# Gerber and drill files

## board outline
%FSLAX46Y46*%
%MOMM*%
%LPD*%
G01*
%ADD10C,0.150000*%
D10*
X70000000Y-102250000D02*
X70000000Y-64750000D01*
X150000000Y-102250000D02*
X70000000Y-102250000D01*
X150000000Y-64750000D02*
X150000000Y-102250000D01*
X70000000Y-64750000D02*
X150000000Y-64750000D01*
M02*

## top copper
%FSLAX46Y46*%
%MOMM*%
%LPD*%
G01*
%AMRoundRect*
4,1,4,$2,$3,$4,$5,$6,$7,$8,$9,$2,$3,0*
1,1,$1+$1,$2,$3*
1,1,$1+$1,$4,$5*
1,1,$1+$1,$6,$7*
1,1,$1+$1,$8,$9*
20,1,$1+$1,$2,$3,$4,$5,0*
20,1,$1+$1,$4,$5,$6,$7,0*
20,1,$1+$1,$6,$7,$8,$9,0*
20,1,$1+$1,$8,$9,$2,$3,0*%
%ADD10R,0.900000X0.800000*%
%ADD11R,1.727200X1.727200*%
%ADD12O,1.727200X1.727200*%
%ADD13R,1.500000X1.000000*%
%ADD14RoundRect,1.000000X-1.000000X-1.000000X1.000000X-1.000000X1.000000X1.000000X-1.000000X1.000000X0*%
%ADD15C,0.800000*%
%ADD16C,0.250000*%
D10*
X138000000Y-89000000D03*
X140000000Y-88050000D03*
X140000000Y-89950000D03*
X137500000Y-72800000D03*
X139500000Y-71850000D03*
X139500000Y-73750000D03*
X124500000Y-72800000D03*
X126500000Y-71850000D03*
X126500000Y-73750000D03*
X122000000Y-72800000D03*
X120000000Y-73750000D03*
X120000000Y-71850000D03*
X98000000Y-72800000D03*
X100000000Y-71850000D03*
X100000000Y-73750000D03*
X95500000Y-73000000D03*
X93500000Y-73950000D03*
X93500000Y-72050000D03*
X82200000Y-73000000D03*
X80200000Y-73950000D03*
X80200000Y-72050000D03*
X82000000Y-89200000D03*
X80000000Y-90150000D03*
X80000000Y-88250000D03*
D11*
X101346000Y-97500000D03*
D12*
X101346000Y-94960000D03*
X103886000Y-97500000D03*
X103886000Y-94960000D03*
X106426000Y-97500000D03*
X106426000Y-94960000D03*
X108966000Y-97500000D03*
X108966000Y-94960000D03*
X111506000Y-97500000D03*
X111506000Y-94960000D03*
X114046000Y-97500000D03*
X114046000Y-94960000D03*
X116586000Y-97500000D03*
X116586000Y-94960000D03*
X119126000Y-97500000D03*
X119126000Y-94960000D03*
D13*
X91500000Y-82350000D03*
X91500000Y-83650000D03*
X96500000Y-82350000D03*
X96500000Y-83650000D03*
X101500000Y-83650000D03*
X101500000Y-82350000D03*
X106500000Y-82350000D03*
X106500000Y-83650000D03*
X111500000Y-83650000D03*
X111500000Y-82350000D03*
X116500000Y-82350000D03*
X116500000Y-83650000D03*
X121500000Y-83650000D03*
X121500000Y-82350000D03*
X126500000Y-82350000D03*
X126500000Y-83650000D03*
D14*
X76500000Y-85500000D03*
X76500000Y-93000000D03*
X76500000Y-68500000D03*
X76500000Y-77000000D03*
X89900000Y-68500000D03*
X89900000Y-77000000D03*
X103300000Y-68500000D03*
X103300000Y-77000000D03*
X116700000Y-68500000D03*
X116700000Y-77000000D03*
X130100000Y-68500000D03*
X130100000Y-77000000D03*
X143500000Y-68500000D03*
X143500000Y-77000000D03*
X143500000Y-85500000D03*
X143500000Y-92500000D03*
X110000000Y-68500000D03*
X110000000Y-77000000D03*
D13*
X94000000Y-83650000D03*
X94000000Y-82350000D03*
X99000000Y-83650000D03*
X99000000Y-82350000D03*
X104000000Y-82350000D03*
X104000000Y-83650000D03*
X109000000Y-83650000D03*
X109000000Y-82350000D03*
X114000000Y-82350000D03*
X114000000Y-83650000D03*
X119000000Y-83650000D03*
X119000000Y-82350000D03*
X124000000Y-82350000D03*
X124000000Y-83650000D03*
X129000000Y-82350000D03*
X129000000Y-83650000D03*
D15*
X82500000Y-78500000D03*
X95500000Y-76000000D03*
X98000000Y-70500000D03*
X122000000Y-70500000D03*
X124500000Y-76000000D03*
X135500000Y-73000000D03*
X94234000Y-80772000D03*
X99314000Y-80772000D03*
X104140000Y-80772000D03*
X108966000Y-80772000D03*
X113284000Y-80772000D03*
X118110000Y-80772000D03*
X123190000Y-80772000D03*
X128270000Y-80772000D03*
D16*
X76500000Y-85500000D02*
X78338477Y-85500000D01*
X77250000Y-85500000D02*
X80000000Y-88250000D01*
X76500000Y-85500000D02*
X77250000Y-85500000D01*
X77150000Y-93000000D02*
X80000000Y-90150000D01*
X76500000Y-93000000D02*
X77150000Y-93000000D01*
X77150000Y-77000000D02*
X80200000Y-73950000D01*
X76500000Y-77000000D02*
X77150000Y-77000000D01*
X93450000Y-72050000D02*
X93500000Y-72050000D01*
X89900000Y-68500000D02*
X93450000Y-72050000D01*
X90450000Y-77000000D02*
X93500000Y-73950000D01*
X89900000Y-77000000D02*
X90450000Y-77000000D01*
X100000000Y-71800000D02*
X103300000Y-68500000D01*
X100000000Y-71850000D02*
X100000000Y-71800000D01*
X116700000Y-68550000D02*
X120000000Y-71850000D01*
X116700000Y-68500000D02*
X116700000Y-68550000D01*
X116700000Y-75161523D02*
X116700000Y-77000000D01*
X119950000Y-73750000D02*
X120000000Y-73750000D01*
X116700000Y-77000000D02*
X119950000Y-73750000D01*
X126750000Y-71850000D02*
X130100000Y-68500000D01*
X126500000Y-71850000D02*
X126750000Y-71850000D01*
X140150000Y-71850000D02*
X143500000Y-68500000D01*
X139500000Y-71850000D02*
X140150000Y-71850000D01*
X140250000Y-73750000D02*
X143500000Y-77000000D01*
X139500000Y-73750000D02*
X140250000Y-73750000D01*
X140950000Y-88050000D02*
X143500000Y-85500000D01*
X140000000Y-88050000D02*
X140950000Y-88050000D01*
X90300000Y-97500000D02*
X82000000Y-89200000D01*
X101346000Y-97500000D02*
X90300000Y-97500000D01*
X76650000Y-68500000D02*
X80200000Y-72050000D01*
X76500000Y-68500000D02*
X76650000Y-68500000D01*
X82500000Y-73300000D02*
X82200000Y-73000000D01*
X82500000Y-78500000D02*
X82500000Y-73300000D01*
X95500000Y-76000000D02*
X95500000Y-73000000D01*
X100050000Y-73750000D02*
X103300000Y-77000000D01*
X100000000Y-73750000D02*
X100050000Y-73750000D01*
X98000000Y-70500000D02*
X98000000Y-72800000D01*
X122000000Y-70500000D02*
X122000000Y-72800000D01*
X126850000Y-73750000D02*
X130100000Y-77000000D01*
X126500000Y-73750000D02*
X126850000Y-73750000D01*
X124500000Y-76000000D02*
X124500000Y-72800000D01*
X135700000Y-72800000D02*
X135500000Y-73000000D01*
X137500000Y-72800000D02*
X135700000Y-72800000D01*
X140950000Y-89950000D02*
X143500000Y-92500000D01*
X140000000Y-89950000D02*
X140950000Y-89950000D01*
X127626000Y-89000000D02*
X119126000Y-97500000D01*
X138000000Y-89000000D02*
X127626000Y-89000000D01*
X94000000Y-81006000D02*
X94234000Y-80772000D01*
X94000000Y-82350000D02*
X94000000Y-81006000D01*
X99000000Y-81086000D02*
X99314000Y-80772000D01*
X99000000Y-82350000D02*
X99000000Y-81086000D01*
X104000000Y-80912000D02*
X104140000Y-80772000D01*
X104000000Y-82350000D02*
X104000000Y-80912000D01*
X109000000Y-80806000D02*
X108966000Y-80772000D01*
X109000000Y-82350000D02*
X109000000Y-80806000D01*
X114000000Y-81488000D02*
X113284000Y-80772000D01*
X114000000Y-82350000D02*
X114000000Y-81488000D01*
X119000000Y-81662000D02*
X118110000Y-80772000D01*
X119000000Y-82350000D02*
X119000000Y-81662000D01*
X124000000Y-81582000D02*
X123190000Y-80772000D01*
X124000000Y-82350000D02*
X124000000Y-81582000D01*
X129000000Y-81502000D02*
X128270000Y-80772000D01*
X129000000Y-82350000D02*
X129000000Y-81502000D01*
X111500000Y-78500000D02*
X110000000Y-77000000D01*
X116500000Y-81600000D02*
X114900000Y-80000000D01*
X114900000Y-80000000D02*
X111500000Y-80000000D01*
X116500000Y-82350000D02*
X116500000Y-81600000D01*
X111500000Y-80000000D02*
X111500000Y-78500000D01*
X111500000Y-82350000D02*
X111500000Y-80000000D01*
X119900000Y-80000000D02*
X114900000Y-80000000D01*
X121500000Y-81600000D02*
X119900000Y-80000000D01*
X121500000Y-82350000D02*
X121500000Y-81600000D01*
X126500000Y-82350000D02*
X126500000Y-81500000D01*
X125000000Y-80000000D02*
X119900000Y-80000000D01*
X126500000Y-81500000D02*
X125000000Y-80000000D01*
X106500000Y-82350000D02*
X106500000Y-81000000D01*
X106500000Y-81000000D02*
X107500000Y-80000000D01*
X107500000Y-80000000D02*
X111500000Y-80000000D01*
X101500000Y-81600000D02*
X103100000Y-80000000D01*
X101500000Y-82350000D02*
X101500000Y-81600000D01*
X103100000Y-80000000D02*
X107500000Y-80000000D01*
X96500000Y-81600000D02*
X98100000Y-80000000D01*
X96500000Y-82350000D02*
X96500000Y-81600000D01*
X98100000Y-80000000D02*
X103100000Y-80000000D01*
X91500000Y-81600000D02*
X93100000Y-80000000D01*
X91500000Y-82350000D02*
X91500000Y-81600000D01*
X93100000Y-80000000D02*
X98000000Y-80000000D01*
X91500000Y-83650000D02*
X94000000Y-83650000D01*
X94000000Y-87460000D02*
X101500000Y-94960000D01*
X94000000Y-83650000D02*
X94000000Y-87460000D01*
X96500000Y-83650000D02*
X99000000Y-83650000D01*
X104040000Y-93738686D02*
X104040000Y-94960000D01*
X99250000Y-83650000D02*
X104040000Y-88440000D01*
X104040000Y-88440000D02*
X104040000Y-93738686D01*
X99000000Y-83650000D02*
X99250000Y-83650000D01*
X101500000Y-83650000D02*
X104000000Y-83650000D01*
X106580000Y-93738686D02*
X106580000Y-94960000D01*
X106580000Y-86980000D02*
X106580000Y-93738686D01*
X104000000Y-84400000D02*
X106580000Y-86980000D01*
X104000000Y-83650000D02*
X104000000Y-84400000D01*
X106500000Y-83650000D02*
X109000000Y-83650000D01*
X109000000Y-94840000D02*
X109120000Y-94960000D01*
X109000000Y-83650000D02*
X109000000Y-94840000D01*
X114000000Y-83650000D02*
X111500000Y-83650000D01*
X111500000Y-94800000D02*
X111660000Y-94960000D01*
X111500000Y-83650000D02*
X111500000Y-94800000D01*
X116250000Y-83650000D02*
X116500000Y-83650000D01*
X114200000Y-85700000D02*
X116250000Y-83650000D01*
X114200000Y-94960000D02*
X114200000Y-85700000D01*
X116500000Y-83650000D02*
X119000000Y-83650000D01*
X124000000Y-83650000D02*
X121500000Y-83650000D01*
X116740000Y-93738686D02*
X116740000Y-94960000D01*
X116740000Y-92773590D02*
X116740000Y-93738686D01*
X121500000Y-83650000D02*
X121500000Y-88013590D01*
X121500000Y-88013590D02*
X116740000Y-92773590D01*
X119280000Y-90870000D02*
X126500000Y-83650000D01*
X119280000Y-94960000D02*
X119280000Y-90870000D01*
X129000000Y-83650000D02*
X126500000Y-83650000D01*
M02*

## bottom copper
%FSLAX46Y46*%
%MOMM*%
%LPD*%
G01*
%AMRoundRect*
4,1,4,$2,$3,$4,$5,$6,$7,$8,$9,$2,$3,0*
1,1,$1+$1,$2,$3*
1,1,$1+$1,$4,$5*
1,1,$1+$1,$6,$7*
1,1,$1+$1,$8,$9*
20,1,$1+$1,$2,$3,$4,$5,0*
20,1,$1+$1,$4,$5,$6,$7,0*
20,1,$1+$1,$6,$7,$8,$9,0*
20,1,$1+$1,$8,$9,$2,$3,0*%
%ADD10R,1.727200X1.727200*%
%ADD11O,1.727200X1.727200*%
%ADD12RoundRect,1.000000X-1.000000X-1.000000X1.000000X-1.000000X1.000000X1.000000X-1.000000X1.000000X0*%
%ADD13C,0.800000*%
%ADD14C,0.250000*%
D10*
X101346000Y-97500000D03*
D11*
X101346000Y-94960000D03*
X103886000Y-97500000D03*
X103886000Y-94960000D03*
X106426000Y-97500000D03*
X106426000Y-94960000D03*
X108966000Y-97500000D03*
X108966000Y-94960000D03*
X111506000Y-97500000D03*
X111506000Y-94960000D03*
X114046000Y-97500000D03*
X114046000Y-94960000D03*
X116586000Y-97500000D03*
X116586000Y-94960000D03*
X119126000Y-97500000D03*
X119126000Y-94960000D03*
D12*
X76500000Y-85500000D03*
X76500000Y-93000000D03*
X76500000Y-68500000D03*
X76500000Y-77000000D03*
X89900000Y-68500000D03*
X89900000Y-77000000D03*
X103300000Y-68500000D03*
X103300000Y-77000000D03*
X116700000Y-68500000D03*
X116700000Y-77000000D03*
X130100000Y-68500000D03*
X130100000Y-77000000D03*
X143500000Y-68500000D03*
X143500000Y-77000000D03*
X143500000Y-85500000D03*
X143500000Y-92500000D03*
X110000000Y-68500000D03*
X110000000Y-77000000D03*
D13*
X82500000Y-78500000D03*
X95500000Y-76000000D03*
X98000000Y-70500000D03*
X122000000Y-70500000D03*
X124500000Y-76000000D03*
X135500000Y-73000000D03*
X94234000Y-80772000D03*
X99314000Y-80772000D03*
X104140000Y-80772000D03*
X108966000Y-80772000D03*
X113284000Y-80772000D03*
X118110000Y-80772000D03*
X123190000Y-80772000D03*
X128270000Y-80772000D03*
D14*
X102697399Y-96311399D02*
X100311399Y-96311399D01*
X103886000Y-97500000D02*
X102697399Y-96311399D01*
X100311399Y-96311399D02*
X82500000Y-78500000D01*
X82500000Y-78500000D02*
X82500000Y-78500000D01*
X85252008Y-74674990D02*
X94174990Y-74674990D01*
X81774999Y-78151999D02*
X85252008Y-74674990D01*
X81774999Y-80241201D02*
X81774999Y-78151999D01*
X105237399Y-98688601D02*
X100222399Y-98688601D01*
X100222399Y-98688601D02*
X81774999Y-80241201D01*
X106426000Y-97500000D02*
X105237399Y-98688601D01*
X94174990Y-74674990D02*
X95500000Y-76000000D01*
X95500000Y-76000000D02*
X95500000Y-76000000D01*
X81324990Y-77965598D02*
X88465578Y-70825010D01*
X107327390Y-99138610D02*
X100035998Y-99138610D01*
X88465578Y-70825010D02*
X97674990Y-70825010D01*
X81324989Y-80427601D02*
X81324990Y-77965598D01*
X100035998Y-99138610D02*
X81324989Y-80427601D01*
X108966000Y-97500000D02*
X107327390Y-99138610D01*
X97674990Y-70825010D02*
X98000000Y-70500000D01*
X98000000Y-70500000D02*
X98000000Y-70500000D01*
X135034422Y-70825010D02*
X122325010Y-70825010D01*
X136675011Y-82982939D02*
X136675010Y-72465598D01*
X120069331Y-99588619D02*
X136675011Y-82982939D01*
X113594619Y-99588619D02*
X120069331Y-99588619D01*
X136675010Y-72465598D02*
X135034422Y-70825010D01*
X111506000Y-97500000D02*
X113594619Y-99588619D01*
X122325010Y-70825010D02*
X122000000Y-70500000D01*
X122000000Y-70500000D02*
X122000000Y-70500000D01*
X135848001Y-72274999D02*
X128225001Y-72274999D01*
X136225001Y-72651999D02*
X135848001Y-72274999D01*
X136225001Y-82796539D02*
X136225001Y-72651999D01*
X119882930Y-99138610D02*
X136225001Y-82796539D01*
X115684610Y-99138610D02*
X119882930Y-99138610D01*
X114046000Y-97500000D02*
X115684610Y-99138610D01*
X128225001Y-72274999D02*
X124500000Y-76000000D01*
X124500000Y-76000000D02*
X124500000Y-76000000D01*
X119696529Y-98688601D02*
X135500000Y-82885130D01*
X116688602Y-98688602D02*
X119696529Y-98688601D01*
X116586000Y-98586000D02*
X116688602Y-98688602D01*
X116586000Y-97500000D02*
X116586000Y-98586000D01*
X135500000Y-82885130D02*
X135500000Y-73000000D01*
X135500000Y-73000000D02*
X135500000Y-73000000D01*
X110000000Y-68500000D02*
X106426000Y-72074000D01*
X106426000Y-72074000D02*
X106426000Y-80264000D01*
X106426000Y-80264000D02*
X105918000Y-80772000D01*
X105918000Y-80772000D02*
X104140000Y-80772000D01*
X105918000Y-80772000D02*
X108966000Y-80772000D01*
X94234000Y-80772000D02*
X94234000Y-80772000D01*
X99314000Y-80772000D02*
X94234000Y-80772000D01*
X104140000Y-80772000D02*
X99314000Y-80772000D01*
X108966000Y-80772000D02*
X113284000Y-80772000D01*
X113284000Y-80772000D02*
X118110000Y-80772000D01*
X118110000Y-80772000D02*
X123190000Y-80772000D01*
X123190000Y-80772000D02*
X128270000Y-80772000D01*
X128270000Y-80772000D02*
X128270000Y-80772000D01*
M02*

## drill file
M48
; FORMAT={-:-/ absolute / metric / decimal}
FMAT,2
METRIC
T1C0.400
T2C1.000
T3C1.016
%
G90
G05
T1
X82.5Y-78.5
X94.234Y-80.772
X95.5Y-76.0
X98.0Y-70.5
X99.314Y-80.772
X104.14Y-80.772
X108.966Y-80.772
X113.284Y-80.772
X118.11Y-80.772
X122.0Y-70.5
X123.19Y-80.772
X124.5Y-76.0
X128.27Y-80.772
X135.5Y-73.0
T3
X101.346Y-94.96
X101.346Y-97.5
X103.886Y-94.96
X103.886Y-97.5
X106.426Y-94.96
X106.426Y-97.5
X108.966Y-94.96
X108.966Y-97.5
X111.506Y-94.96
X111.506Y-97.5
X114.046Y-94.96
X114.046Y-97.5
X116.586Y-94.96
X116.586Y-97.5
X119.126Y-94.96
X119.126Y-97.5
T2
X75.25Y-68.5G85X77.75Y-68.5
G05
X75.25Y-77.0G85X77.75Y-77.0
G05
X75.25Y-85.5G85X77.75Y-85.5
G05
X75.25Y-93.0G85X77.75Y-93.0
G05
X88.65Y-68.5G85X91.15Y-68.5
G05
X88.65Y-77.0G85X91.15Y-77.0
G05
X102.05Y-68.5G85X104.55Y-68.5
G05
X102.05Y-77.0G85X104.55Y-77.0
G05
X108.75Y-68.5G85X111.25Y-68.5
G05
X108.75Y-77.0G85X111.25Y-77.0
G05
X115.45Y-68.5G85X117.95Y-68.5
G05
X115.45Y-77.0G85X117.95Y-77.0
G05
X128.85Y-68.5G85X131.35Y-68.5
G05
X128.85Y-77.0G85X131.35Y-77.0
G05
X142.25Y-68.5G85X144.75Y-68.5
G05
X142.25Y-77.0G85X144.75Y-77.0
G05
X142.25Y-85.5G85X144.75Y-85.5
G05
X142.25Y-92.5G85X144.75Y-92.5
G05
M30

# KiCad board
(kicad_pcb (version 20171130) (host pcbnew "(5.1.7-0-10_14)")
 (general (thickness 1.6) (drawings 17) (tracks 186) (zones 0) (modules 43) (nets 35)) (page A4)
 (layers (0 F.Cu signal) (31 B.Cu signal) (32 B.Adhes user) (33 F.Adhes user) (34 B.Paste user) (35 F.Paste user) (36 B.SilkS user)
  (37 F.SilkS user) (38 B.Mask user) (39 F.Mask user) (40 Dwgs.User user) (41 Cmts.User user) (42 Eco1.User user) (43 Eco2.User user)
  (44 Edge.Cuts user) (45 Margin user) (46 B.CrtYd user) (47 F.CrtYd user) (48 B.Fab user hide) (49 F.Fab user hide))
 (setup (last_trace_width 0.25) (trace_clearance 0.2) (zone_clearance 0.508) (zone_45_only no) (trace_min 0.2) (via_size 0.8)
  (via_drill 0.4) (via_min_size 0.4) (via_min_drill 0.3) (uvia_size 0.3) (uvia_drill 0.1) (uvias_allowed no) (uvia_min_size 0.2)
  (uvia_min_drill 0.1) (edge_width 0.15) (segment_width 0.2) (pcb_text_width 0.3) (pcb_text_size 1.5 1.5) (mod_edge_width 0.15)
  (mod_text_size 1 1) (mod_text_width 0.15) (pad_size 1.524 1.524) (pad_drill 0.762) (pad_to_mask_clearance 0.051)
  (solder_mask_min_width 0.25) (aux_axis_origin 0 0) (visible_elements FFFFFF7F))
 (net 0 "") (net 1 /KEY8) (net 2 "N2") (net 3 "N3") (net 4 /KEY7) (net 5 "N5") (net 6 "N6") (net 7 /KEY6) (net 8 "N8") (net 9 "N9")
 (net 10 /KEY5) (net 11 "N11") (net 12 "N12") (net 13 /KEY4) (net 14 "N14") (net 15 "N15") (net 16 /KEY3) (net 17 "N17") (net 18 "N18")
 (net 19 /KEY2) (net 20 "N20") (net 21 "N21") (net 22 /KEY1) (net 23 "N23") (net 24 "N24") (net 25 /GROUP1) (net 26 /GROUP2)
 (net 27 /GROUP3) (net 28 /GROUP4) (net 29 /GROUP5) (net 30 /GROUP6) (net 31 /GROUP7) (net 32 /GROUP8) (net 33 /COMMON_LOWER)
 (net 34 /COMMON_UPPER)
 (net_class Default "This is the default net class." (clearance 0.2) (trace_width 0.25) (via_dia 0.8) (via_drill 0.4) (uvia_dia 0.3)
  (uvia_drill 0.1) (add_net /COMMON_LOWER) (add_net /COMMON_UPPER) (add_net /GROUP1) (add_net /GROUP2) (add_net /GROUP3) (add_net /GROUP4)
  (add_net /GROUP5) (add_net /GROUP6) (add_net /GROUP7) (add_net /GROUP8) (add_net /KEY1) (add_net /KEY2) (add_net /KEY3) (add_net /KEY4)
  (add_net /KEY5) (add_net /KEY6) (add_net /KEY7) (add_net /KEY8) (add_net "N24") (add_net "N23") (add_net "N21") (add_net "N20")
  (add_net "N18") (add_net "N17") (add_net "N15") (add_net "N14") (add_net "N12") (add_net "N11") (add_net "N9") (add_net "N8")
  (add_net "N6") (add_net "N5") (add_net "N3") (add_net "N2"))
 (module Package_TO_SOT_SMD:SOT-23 (layer F.Cu) (at 139 89 180)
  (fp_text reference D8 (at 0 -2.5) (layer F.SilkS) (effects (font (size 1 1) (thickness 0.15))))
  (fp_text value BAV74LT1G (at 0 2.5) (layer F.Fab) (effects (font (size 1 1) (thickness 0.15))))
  (pad 3 smd rect (at 1 0 180) (size 0.9 0.8) (layers F.Cu F.Paste F.Mask) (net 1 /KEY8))
  (pad 2 smd rect (at -1 0.95 180) (size 0.9 0.8) (layers F.Cu F.Paste F.Mask) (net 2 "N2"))
  (pad 1 smd rect (at -1 -0.95 180) (size 0.9 0.8) (layers F.Cu F.Paste F.Mask) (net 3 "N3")))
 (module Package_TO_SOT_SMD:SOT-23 (layer F.Cu) (at 138.5 72.8 180)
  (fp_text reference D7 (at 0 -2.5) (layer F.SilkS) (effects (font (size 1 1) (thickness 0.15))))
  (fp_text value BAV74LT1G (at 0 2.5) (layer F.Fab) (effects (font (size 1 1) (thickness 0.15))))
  (pad 3 smd rect (at 1 0 180) (size 0.9 0.8) (layers F.Cu F.Paste F.Mask) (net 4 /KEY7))
  (pad 2 smd rect (at -1 0.95 180) (size 0.9 0.8) (layers F.Cu F.Paste F.Mask) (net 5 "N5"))
  (pad 1 smd rect (at -1 -0.95 180) (size 0.9 0.8) (layers F.Cu F.Paste F.Mask) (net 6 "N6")))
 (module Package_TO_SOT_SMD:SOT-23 (layer F.Cu) (at 125.5 72.8 180)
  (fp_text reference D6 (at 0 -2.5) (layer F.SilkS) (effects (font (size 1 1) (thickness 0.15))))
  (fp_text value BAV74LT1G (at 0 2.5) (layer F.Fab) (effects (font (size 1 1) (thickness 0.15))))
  (pad 3 smd rect (at 1 0 180) (size 0.9 0.8) (layers F.Cu F.Paste F.Mask) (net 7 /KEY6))
  (pad 2 smd rect (at -1 0.95 180) (size 0.9 0.8) (layers F.Cu F.Paste F.Mask) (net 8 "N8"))
  (pad 1 smd rect (at -1 -0.95 180) (size 0.9 0.8) (layers F.Cu F.Paste F.Mask) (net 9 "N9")))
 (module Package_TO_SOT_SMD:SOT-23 (layer F.Cu) (at 121 72.8)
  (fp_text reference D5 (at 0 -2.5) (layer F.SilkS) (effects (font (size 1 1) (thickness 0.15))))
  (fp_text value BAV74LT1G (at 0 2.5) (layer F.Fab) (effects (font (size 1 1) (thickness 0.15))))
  (pad 3 smd rect (at 1 0) (size 0.9 0.8) (layers F.Cu F.Paste F.Mask) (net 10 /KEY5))
  (pad 2 smd rect (at -1 0.95) (size 0.9 0.8) (layers F.Cu F.Paste F.Mask) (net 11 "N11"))
  (pad 1 smd rect (at -1 -0.95) (size 0.9 0.8) (layers F.Cu F.Paste F.Mask) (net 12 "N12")))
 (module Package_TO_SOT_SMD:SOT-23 (layer F.Cu) (at 99 72.8 180)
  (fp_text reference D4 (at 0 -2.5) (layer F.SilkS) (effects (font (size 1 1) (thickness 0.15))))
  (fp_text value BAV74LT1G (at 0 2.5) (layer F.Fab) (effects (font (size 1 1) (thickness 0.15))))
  (pad 3 smd rect (at 1 0 180) (size 0.9 0.8) (layers F.Cu F.Paste F.Mask) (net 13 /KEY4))
  (pad 2 smd rect (at -1 0.95 180) (size 0.9 0.8) (layers F.Cu F.Paste F.Mask) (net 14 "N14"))
  (pad 1 smd rect (at -1 -0.95 180) (size 0.9 0.8) (layers F.Cu F.Paste F.Mask) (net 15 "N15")))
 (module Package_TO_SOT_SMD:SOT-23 (layer F.Cu) (at 94.5 73)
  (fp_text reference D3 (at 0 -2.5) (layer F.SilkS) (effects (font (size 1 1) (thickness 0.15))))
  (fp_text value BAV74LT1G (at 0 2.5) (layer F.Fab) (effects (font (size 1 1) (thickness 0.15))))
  (pad 3 smd rect (at 1 0) (size 0.9 0.8) (layers F.Cu F.Paste F.Mask) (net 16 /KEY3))
  (pad 2 smd rect (at -1 0.95) (size 0.9 0.8) (layers F.Cu F.Paste F.Mask) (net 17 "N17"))
  (pad 1 smd rect (at -1 -0.95) (size 0.9 0.8) (layers F.Cu F.Paste F.Mask) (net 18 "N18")))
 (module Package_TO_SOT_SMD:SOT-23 (layer F.Cu) (at 81.2 73)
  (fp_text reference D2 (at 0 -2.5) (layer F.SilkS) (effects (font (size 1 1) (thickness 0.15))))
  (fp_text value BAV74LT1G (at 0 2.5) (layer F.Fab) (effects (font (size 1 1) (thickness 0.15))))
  (pad 3 smd rect (at 1 0) (size 0.9 0.8) (layers F.Cu F.Paste F.Mask) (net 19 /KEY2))
  (pad 2 smd rect (at -1 0.95) (size 0.9 0.8) (layers F.Cu F.Paste F.Mask) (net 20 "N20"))
  (pad 1 smd rect (at -1 -0.95) (size 0.9 0.8) (layers F.Cu F.Paste F.Mask) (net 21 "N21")))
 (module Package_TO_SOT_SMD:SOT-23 (layer F.Cu) (at 81 89.2)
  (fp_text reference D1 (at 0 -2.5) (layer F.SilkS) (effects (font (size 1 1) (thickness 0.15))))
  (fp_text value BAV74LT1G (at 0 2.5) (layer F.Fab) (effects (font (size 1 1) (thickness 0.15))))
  (pad 3 smd rect (at 1 0) (size 0.9 0.8) (layers F.Cu F.Paste F.Mask) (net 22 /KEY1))
  (pad 2 smd rect (at -1 0.95) (size 0.9 0.8) (layers F.Cu F.Paste F.Mask) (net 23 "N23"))
  (pad 1 smd rect (at -1 -0.95) (size 0.9 0.8) (layers F.Cu F.Paste F.Mask) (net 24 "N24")))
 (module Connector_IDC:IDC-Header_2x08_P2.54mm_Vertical (layer F.Cu) (at 101.346 97.5 90)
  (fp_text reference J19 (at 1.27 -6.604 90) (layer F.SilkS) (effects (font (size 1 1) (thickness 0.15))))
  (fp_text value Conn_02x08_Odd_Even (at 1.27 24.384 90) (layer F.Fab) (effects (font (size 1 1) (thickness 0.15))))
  (pad 1 thru_hole rect (at 0 0 90) (size 1.7272 1.7272) (drill 1.016) (layers *.Cu *.Mask) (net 22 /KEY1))
  (pad 2 thru_hole oval (at 2.54 0 90) (size 1.7272 1.7272) (drill 1.016) (layers *.Cu *.Mask) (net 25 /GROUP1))
  (pad 3 thru_hole oval (at 0 2.54 90) (size 1.7272 1.7272) (drill 1.016) (layers *.Cu *.Mask) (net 19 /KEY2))
  (pad 4 thru_hole oval (at 2.54 2.54 90) (size 1.7272 1.7272) (drill 1.016) (layers *.Cu *.Mask) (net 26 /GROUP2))
  (pad 5 thru_hole oval (at 0 5.08 90) (size 1.7272 1.7272) (drill 1.016) (layers *.Cu *.Mask) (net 16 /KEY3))
  (pad 6 thru_hole oval (at 2.54 5.08 90) (size 1.7272 1.7272) (drill 1.016) (layers *.Cu *.Mask) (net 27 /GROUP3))
  (pad 7 thru_hole oval (at 0 7.62 90) (size 1.7272 1.7272) (drill 1.016) (layers *.Cu *.Mask) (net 13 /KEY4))
  (pad 8 thru_hole oval (at 2.54 7.62 90) (size 1.7272 1.7272) (drill 1.016) (layers *.Cu *.Mask) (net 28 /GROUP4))
  (pad 9 thru_hole oval (at 0 10.16 90) (size 1.7272 1.7272) (drill 1.016) (layers *.Cu *.Mask) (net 10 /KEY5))
  (pad 10 thru_hole oval (at 2.54 10.16 90) (size 1.7272 1.7272) (drill 1.016) (layers *.Cu *.Mask) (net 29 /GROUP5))
  (pad 11 thru_hole oval (at 0 12.7 90) (size 1.7272 1.7272) (drill 1.016) (layers *.Cu *.Mask) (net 7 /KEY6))
  (pad 12 thru_hole oval (at 2.54 12.7 90) (size 1.7272 1.7272) (drill 1.016) (layers *.Cu *.Mask) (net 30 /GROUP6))
  (pad 13 thru_hole oval (at 0 15.24 90) (size 1.7272 1.7272) (drill 1.016) (layers *.Cu *.Mask) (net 4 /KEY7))
  (pad 14 thru_hole oval (at 2.54 15.24 90) (size 1.7272 1.7272) (drill 1.016) (layers *.Cu *.Mask) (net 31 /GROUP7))
  (pad 15 thru_hole oval (at 0 17.78 90) (size 1.7272 1.7272) (drill 1.016) (layers *.Cu *.Mask) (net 1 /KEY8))
  (pad 16 thru_hole oval (at 2.54 17.78 90) (size 1.7272 1.7272) (drill 1.016) (layers *.Cu *.Mask) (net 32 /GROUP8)))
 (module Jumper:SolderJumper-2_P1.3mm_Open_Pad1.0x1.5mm (layer F.Cu) (at 91.5 83 90)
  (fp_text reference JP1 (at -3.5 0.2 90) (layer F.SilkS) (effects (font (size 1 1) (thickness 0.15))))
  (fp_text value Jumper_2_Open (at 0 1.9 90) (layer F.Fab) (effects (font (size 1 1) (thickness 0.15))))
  (pad 2 smd rect (at 0.65 0 90) (size 1 1.5) (layers F.Cu F.Mask) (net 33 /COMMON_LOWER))
  (pad 1 smd rect (at -0.65 0 90) (size 1 1.5) (layers F.Cu F.Mask) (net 25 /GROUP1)))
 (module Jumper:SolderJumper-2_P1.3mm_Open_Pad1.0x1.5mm (layer F.Cu) (at 96.5 83 90)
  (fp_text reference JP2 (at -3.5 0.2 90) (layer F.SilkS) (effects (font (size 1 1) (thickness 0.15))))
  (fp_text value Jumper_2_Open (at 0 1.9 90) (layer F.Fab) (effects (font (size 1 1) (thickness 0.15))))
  (pad 2 smd rect (at 0.65 0 90) (size 1 1.5) (layers F.Cu F.Mask) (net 33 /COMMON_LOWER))
  (pad 1 smd rect (at -0.65 0 90) (size 1 1.5) (layers F.Cu F.Mask) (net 26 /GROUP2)))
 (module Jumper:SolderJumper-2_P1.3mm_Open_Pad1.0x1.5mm (layer F.Cu) (at 101.5 83 90)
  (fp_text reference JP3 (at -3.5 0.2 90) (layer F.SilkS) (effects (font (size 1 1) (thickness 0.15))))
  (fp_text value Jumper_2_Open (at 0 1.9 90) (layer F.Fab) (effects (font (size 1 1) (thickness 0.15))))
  (pad 1 smd rect (at -0.65 0 90) (size 1 1.5) (layers F.Cu F.Mask) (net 27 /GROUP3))
  (pad 2 smd rect (at 0.65 0 90) (size 1 1.5) (layers F.Cu F.Mask) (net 33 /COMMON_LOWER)))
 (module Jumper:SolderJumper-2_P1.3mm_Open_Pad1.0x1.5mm (layer F.Cu) (at 106.5 83 90)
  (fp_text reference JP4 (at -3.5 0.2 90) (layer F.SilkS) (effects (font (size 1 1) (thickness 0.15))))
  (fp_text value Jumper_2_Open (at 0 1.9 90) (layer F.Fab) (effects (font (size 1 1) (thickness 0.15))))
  (pad 2 smd rect (at 0.65 0 90) (size 1 1.5) (layers F.Cu F.Mask) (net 33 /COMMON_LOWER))
  (pad 1 smd rect (at -0.65 0 90) (size 1 1.5) (layers F.Cu F.Mask) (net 28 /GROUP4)))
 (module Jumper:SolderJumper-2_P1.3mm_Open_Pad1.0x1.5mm (layer F.Cu) (at 111.5 83 90)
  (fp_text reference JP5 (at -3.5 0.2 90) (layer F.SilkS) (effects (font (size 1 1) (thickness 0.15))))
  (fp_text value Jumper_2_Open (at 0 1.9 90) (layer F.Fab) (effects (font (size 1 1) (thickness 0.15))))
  (pad 1 smd rect (at -0.65 0 90) (size 1 1.5) (layers F.Cu F.Mask) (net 29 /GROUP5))
  (pad 2 smd rect (at 0.65 0 90) (size 1 1.5) (layers F.Cu F.Mask) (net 33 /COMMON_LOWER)))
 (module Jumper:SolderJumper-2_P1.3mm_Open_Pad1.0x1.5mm (layer F.Cu) (at 116.5 83 90)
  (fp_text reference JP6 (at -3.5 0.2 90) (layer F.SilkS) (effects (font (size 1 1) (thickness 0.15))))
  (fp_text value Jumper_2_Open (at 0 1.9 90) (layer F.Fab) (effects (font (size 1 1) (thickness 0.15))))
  (pad 2 smd rect (at 0.65 0 90) (size 1 1.5) (layers F.Cu F.Mask) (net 33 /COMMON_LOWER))
  (pad 1 smd rect (at -0.65 0 90) (size 1 1.5) (layers F.Cu F.Mask) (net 30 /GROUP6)))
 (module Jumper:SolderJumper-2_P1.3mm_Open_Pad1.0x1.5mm (layer F.Cu) (at 121.5 83 90)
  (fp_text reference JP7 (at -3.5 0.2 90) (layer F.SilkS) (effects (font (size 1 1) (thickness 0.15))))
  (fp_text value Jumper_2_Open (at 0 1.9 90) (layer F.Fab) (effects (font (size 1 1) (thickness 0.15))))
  (pad 1 smd rect (at -0.65 0 90) (size 1 1.5) (layers F.Cu F.Mask) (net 31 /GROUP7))
  (pad 2 smd rect (at 0.65 0 90) (size 1 1.5) (layers F.Cu F.Mask) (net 33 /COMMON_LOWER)))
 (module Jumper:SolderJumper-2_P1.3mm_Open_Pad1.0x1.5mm (layer F.Cu) (at 126.5 83 90)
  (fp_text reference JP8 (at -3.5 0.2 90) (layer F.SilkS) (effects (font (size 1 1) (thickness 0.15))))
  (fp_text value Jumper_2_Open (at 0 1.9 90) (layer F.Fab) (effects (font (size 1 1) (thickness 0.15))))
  (pad 2 smd rect (at 0.65 0 90) (size 1 1.5) (layers F.Cu F.Mask) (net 33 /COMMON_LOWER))
  (pad 1 smd rect (at -0.65 0 90) (size 1 1.5) (layers F.Cu F.Mask) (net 32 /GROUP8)))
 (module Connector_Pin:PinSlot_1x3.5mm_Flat (layer F.Cu) (at 76.5 85.5)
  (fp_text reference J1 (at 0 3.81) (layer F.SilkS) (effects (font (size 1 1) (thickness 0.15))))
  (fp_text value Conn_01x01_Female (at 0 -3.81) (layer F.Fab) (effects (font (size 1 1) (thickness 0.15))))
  (pad 1 thru_hole roundrect (at 0 0) (size 4 4) (drill oval 3.5 1) (layers *.Cu *.Mask) (roundrect_rratio 0.25) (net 24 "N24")))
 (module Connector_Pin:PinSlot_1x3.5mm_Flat (layer F.Cu) (at 76.5 93)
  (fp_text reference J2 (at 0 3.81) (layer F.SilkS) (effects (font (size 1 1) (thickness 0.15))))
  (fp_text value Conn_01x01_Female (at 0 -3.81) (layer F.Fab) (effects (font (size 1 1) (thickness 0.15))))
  (pad 1 thru_hole roundrect (at 0 0) (size 4 4) (drill oval 3.5 1) (layers *.Cu *.Mask) (roundrect_rratio 0.25) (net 23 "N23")))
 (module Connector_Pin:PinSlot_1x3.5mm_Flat (layer F.Cu) (at 76.5 68.5)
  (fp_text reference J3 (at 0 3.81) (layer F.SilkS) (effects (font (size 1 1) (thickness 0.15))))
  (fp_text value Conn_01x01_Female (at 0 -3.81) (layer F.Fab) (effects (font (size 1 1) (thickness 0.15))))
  (pad 1 thru_hole roundrect (at 0 0) (size 4 4) (drill oval 3.5 1) (layers *.Cu *.Mask) (roundrect_rratio 0.25) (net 21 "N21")))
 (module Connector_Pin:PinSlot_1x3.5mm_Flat (layer F.Cu) (at 76.5 77)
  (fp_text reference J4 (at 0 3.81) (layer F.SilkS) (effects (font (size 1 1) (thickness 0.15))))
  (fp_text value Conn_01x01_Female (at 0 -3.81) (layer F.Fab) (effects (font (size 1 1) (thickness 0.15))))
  (pad 1 thru_hole roundrect (at 0 0) (size 4 4) (drill oval 3.5 1) (layers *.Cu *.Mask) (roundrect_rratio 0.25) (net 20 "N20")))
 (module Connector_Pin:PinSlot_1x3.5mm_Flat (layer F.Cu) (at 89.9 68.5)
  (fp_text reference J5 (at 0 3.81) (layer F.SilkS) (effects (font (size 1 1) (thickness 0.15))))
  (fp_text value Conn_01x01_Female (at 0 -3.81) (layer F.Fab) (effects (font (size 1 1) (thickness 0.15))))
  (pad 1 thru_hole roundrect (at 0 0) (size 4 4) (drill oval 3.5 1) (layers *.Cu *.Mask) (roundrect_rratio 0.25) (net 18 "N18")))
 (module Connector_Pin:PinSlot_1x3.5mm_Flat (layer F.Cu) (at 89.9 77)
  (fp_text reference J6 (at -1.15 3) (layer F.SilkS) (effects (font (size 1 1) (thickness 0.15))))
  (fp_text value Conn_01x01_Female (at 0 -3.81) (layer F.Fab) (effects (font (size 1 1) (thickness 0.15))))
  (pad 1 thru_hole roundrect (at 0 0) (size 4 4) (drill oval 3.5 1) (layers *.Cu *.Mask) (roundrect_rratio 0.25) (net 17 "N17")))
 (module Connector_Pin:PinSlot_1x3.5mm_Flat (layer F.Cu) (at 103.3 68.5)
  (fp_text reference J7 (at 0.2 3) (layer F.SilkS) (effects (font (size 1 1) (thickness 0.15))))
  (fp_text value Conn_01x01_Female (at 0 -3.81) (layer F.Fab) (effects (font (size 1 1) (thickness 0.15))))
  (pad 1 thru_hole roundrect (at 0 0) (size 4 4) (drill oval 3.5 1) (layers *.Cu *.Mask) (roundrect_rratio 0.25) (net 14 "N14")))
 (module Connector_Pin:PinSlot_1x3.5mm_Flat (layer F.Cu) (at 103.3 77)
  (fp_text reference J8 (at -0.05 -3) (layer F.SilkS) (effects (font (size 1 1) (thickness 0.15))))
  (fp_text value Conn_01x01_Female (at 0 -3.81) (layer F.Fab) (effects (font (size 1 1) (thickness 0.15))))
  (pad 1 thru_hole roundrect (at 0 0) (size 4 4) (drill oval 3.5 1) (layers *.Cu *.Mask) (roundrect_rratio 0.25) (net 15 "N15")))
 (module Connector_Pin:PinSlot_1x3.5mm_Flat (layer F.Cu) (at 116.7 68.5)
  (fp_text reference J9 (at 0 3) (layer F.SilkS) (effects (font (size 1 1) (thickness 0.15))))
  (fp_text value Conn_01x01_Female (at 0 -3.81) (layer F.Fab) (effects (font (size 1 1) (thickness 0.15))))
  (pad 1 thru_hole roundrect (at 0 0) (size 4 4) (drill oval 3.5 1) (layers *.Cu *.Mask) (roundrect_rratio 0.25) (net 12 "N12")))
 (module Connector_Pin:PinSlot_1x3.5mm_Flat (layer F.Cu) (at 116.7 77)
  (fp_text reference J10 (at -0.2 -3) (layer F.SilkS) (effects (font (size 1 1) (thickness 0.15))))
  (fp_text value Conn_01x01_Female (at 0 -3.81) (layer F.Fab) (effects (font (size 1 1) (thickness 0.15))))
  (pad 1 thru_hole roundrect (at 0 0) (size 4 4) (drill oval 3.5 1) (layers *.Cu *.Mask) (roundrect_rratio 0.25) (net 11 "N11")))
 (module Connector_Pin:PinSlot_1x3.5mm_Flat (layer F.Cu) (at 130.1 68.5)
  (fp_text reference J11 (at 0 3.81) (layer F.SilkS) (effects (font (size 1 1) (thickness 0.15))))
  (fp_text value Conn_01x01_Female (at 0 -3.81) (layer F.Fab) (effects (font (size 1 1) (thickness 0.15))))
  (pad 1 thru_hole roundrect (at 0 0) (size 4 4) (drill oval 3.5 1) (layers *.Cu *.Mask) (roundrect_rratio 0.25) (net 8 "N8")))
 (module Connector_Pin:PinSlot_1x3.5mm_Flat (layer F.Cu) (at 130.1 77)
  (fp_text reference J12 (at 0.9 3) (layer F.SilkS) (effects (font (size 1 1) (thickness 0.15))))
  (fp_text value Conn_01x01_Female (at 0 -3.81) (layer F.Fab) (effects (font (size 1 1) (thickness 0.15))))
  (pad 1 thru_hole roundrect (at 0 0) (size 4 4) (drill oval 3.5 1) (layers *.Cu *.Mask) (roundrect_rratio 0.25) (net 9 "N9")))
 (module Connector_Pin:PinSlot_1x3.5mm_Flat (layer F.Cu) (at 143.5 68.5)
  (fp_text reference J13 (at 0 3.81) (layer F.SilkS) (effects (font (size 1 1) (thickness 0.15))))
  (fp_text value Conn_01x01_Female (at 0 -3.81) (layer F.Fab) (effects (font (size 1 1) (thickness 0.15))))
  (pad 1 thru_hole roundrect (at 0 0) (size 4 4) (drill oval 3.5 1) (layers *.Cu *.Mask) (roundrect_rratio 0.25) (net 5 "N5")))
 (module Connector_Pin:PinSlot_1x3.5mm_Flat (layer F.Cu) (at 143.5 77)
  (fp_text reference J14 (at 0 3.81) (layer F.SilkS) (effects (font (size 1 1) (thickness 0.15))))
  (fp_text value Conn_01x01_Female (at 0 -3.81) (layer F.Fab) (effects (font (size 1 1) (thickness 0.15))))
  (pad 1 thru_hole roundrect (at 0 0) (size 4 4) (drill oval 3.5 1) (layers *.Cu *.Mask) (roundrect_rratio 0.25) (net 6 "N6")))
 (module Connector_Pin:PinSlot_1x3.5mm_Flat (layer F.Cu) (at 143.5 85.5)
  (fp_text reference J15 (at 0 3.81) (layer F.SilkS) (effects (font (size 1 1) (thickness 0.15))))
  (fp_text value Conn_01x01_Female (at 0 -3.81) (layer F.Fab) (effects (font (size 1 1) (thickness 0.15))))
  (pad 1 thru_hole roundrect (at 0 0) (size 4 4) (drill oval 3.5 1) (layers *.Cu *.Mask) (roundrect_rratio 0.25) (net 2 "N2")))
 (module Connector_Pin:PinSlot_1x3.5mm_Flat (layer F.Cu) (at 143.5 92.5)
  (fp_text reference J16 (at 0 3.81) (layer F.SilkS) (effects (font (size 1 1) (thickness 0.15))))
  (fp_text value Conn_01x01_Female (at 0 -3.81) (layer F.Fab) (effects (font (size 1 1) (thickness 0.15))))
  (pad 1 thru_hole roundrect (at 0 0) (size 4 4) (drill oval 3.5 1) (layers *.Cu *.Mask) (roundrect_rratio 0.25) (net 3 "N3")))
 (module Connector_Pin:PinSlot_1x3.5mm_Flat (layer F.Cu) (at 110 68.5)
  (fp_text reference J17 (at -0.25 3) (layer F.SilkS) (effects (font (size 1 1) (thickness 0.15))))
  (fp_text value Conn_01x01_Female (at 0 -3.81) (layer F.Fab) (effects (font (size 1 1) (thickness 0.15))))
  (pad 1 thru_hole roundrect (at 0 0) (size 4 4) (drill oval 3.5 1) (layers *.Cu *.Mask) (roundrect_rratio 0.25) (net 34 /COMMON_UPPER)))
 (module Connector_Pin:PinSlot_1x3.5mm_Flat (layer F.Cu) (at 110 77)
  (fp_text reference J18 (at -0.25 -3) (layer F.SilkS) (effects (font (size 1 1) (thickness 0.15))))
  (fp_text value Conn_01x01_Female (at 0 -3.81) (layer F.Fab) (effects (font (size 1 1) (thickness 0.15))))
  (pad 1 thru_hole roundrect (at 0 0) (size 4 4) (drill oval 3.5 1) (layers *.Cu *.Mask) (roundrect_rratio 0.25) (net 33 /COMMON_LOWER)))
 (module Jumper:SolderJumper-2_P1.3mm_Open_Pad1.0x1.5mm (layer F.Cu) (at 94 83 90)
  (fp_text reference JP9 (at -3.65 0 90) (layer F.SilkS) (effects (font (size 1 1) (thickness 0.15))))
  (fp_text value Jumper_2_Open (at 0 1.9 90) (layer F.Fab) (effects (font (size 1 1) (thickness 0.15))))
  (pad 1 smd rect (at -0.65 0 90) (size 1 1.5) (layers F.Cu F.Mask) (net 25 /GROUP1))
  (pad 2 smd rect (at 0.65 0 90) (size 1 1.5) (layers F.Cu F.Mask) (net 34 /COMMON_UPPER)))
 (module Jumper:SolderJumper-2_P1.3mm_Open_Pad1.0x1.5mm (layer F.Cu) (at 99 83 90)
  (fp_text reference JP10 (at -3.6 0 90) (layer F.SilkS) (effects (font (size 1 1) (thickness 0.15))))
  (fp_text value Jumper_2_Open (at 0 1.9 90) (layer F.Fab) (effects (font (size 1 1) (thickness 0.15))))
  (pad 1 smd rect (at -0.65 0 90) (size 1 1.5) (layers F.Cu F.Mask) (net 26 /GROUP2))
  (pad 2 smd rect (at 0.65 0 90) (size 1 1.5) (layers F.Cu F.Mask) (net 34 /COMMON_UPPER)))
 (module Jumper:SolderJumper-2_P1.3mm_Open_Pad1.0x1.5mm (layer F.Cu) (at 104 83 90)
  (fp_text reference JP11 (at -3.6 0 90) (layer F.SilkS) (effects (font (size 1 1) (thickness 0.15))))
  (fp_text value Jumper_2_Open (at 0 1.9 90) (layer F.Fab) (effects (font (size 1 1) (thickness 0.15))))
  (pad 2 smd rect (at 0.65 0 90) (size 1 1.5) (layers F.Cu F.Mask) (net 34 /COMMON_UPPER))
  (pad 1 smd rect (at -0.65 0 90) (size 1 1.5) (layers F.Cu F.Mask) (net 27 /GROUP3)))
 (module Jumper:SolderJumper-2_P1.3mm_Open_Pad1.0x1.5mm (layer F.Cu) (at 109 83 90)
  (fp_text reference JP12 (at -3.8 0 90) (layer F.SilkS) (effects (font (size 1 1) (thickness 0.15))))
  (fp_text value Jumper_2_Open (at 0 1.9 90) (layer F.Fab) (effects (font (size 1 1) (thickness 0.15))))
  (pad 1 smd rect (at -0.65 0 90) (size 1 1.5) (layers F.Cu F.Mask) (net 28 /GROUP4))
  (pad 2 smd rect (at 0.65 0 90) (size 1 1.5) (layers F.Cu F.Mask) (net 34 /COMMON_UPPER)))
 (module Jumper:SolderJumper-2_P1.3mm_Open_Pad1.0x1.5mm (layer F.Cu) (at 114 83 90)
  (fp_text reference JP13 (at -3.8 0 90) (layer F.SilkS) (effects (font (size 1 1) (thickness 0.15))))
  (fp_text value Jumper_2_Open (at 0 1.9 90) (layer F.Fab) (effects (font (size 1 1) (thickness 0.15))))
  (pad 2 smd rect (at 0.65 0 90) (size 1 1.5) (layers F.Cu F.Mask) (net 34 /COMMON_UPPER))
  (pad 1 smd rect (at -0.65 0 90) (size 1 1.5) (layers F.Cu F.Mask) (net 29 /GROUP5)))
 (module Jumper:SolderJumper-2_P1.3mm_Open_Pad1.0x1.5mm (layer F.Cu) (at 119 83 90)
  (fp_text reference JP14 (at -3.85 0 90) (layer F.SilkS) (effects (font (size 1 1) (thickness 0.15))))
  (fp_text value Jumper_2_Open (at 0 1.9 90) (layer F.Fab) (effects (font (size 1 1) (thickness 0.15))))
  (pad 1 smd rect (at -0.65 0 90) (size 1 1.5) (layers F.Cu F.Mask) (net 30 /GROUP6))
  (pad 2 smd rect (at 0.65 0 90) (size 1 1.5) (layers F.Cu F.Mask) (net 34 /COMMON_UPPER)))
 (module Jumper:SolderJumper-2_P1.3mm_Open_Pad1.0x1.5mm (layer F.Cu) (at 124 83 90)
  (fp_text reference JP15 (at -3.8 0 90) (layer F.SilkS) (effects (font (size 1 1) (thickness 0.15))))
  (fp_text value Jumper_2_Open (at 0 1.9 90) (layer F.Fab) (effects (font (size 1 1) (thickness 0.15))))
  (pad 2 smd rect (at 0.65 0 90) (size 1 1.5) (layers F.Cu F.Mask) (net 34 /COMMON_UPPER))
  (pad 1 smd rect (at -0.65 0 90) (size 1 1.5) (layers F.Cu F.Mask) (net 31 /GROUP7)))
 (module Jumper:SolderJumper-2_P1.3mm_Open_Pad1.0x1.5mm (layer F.Cu) (at 129 83 90)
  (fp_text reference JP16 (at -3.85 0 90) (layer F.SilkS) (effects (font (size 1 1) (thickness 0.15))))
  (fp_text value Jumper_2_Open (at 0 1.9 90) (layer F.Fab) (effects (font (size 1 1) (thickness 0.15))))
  (pad 2 smd rect (at 0.65 0 90) (size 1 1.5) (layers F.Cu F.Mask) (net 34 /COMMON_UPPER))
  (pad 1 smd rect (at -0.65 0 90) (size 1 1.5) (layers F.Cu F.Mask) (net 32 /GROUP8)))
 (gr_line (start 70 102.25) (end 70 64.75) (layer Edge.Cuts) (width 0.15))
 (gr_line (start 150 102.25) (end 70 102.25) (layer Edge.Cuts) (width 0.15))
 (gr_line (start 150 64.75) (end 150 102.25) (layer Edge.Cuts) (width 0.15))
 (gr_line (start 70 64.75) (end 150 64.75) (layer Edge.Cuts) (width 0.15))
 (segment (start 76.5 85.5) (end 78.338477 85.5) (width 0.25) (layer F.Cu) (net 24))
 (segment (start 77.25 85.5) (end 80 88.25) (width 0.25) (layer F.Cu) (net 24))
 (segment (start 76.5 85.5) (end 77.25 85.5) (width 0.25) (layer F.Cu) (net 24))
 (segment (start 77.15 93) (end 80 90.15) (width 0.25) (layer F.Cu) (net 23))
 (segment (start 76.5 93) (end 77.15 93) (width 0.25) (layer F.Cu) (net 23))
 (segment (start 77.15 77) (end 80.2 73.95) (width 0.25) (layer F.Cu) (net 20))
 (segment (start 76.5 77) (end 77.15 77) (width 0.25) (layer F.Cu) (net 20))
 (segment (start 93.45 72.05) (end 93.5 72.05) (width 0.25) (layer F.Cu) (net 18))
 (segment (start 89.9 68.5) (end 93.45 72.05) (width 0.25) (layer F.Cu) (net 18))
 (segment (start 90.45 77) (end 93.5 73.95) (width 0.25) (layer F.Cu) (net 17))
 (segment (start 89.9 77) (end 90.45 77) (width 0.25) (layer F.Cu) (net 17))
 (segment (start 100 71.8) (end 103.3 68.5) (width 0.25) (layer F.Cu) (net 14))
 (segment (start 100 71.85) (end 100 71.8) (width 0.25) (layer F.Cu) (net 14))
 (segment (start 116.7 68.55) (end 120 71.85) (width 0.25) (layer F.Cu) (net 12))
 (segment (start 116.7 68.5) (end 116.7 68.55) (width 0.25) (layer F.Cu) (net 12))
 (segment (start 116.7 75.161523) (end 116.7 77) (width 0.25) (layer F.Cu) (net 11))
 (segment (start 119.95 73.75) (end 120 73.75) (width 0.25) (layer F.Cu) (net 11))
 (segment (start 116.7 77) (end 119.95 73.75) (width 0.25) (layer F.Cu) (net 11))
 (segment (start 126.75 71.85) (end 130.1 68.5) (width 0.25) (layer F.Cu) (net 8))
 (segment (start 126.5 71.85) (end 126.75 71.85) (width 0.25) (layer F.Cu) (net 8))
 (segment (start 140.15 71.85) (end 143.5 68.5) (width 0.25) (layer F.Cu) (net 5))
 (segment (start 139.5 71.85) (end 140.15 71.85) (width 0.25) (layer F.Cu) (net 5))
 (segment (start 140.25 73.75) (end 143.5 77) (width 0.25) (layer F.Cu) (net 6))
 (segment (start 139.5 73.75) (end 140.25 73.75) (width 0.25) (layer F.Cu) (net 6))
 (segment (start 140.95 88.05) (end 143.5 85.5) (width 0.25) (layer F.Cu) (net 2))
 (segment (start 140 88.05) (end 140.95 88.05) (width 0.25) (layer F.Cu) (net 2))
 (segment (start 90.3 97.5) (end 82 89.2) (width 0.25) (layer F.Cu) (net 22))
 (segment (start 101.346 97.5) (end 90.3 97.5) (width 0.25) (layer F.Cu) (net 22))
 (segment (start 76.65 68.5) (end 80.2 72.05) (width 0.25) (layer F.Cu) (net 21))
 (segment (start 76.5 68.5) (end 76.65 68.5) (width 0.25) (layer F.Cu) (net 21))
 (segment (start 102.697399 96.311399) (end 100.311399 96.311399) (width 0.25) (layer B.Cu) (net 19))
 (segment (start 103.886 97.5) (end 102.697399 96.311399) (width 0.25) (layer B.Cu) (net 19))
 (segment (start 100.311399 96.311399) (end 82.5 78.5) (width 0.25) (layer B.Cu) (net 19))
 (segment (start 82.5 78.5) (end 82.5 78.5) (width 0.25) (layer B.Cu) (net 19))
 (via (at 82.5 78.5) (size 0.8) (drill 0.4) (layers F.Cu B.Cu) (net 19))
 (segment (start 82.5 73.3) (end 82.2 73) (width 0.25) (layer F.Cu) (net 19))
 (segment (start 82.5 78.5) (end 82.5 73.3) (width 0.25) (layer F.Cu) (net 19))
 (segment (start 85.252008 74.67499) (end 94.17499 74.67499) (width 0.25) (layer B.Cu) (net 16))
 (segment (start 81.774999 78.151999) (end 85.252008 74.67499) (width 0.25) (layer B.Cu) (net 16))
 (segment (start 81.774999 80.241201) (end 81.774999 78.151999) (width 0.25) (layer B.Cu) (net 16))
 (segment (start 105.237399 98.688601) (end 100.222399 98.688601) (width 0.25) (layer B.Cu) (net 16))
 (segment (start 100.222399 98.688601) (end 81.774999 80.241201) (width 0.25) (layer B.Cu) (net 16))
 (segment (start 106.426 97.5) (end 105.237399 98.688601) (width 0.25) (layer B.Cu) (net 16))
 (segment (start 94.17499 74.67499) (end 95.5 76) (width 0.25) (layer B.Cu) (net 16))
 (segment (start 95.5 76) (end 95.5 76) (width 0.25) (layer B.Cu) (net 16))
 (via (at 95.5 76) (size 0.8) (drill 0.4) (layers F.Cu B.Cu) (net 16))
 (segment (start 95.5 76) (end 95.5 73) (width 0.25) (layer F.Cu) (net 16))
 (segment (start 100.05 73.75) (end 103.3 77) (width 0.25) (layer F.Cu) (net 15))
 (segment (start 100 73.75) (end 100.05 73.75) (width 0.25) (layer F.Cu) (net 15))
 (segment (start 81.32499 77.965598) (end 88.465578 70.82501) (width 0.25) (layer B.Cu) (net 13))
 (segment (start 107.32739 99.13861) (end 100.035998 99.13861) (width 0.25) (layer B.Cu) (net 13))
 (segment (start 88.465578 70.82501) (end 97.67499 70.82501) (width 0.25) (layer B.Cu) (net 13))
 (segment (start 81.324989 80.427601) (end 81.32499 77.965598) (width 0.25) (layer B.Cu) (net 13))
 (segment (start 100.035998 99.13861) (end 81.324989 80.427601) (width 0.25) (layer B.Cu) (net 13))
 (segment (start 108.966 97.5) (end 107.32739 99.13861) (width 0.25) (layer B.Cu) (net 13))
 (segment (start 97.67499 70.82501) (end 98 70.5) (width 0.25) (layer B.Cu) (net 13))
 (segment (start 98 70.5) (end 98 70.5) (width 0.25) (layer B.Cu) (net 13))
 (via (at 98 70.5) (size 0.8) (drill 0.4) (layers F.Cu B.Cu) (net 13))
 (segment (start 98 70.5) (end 98 72.8) (width 0.25) (layer F.Cu) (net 13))
 (segment (start 135.034422 70.82501) (end 122.32501 70.82501) (width 0.25) (layer B.Cu) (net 10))
 (segment (start 136.675011 82.982939) (end 136.67501 72.465598) (width 0.25) (layer B.Cu) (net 10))
 (segment (start 120.069331 99.588619) (end 136.675011 82.982939) (width 0.25) (layer B.Cu) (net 10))
 (segment (start 113.594619 99.588619) (end 120.069331 99.588619) (width 0.25) (layer B.Cu) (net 10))
 (segment (start 136.67501 72.465598) (end 135.034422 70.82501) (width 0.25) (layer B.Cu) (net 10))
 (segment (start 111.506 97.5) (end 113.594619 99.588619) (width 0.25) (layer B.Cu) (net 10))
 (segment (start 122.32501 70.82501) (end 122 70.5) (width 0.25) (layer B.Cu) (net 10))
 (segment (start 122 70.5) (end 122 70.5) (width 0.25) (layer B.Cu) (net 10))
 (via (at 122 70.5) (size 0.8) (drill 0.4) (layers F.Cu B.Cu) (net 10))
 (segment (start 122 70.5) (end 122 72.8) (width 0.25) (layer F.Cu) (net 10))
 (segment (start 126.85 73.75) (end 130.1 77) (width 0.25) (layer F.Cu) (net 9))
 (segment (start 126.5 73.75) (end 126.85 73.75) (width 0.25) (layer F.Cu) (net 9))
 (segment (start 135.848001 72.274999) (end 128.225001 72.274999) (width 0.25) (layer B.Cu) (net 7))
 (segment (start 136.225001 72.651999) (end 135.848001 72.274999) (width 0.25) (layer B.Cu) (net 7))
 (segment (start 136.225001 82.796539) (end 136.225001 72.651999) (width 0.25) (layer B.Cu) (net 7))
 (segment (start 119.88293 99.13861) (end 136.225001 82.796539) (width 0.25) (layer B.Cu) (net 7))
 (segment (start 115.68461 99.13861) (end 119.88293 99.13861) (width 0.25) (layer B.Cu) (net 7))
 (segment (start 114.046 97.5) (end 115.68461 99.13861) (width 0.25) (layer B.Cu) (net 7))
 (segment (start 128.225001 72.274999) (end 124.5 76) (width 0.25) (layer B.Cu) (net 7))
 (segment (start 124.5 76) (end 124.5 76) (width 0.25) (layer B.Cu) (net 7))
 (via (at 124.5 76) (size 0.8) (drill 0.4) (layers F.Cu B.Cu) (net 7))
 (segment (start 124.5 76) (end 124.5 72.8) (width 0.25) (layer F.Cu) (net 7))
 (segment (start 119.696529 98.688601) (end 135.5 82.88513) (width 0.25) (layer B.Cu) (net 4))
 (segment (start 116.688602 98.688602) (end 119.696529 98.688601) (width 0.25) (layer B.Cu) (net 4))
 (segment (start 116.586 98.586) (end 116.688602 98.688602) (width 0.25) (layer B.Cu) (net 4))
 (segment (start 116.586 97.5) (end 116.586 98.586) (width 0.25) (layer B.Cu) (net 4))
 (segment (start 135.5 82.88513) (end 135.5 73) (width 0.25) (layer B.Cu) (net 4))
 (segment (start 135.5 73) (end 135.5 73) (width 0.25) (layer B.Cu) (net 4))
 (via (at 135.5 73) (size 0.8) (drill 0.4) (layers F.Cu B.Cu) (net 4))
 (segment (start 135.7 72.8) (end 135.5 73) (width 0.25) (layer F.Cu) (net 4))
 (segment (start 137.5 72.8) (end 135.7 72.8) (width 0.25) (layer F.Cu) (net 4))
 (segment (start 140.95 89.95) (end 143.5 92.5) (width 0.25) (layer F.Cu) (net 3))
 (segment (start 140 89.95) (end 140.95 89.95) (width 0.25) (layer F.Cu) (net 3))
 (segment (start 127.626 89) (end 119.126 97.5) (width 0.25) (layer F.Cu) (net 1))
 (segment (start 138 89) (end 127.626 89) (width 0.25) (layer F.Cu) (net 1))
 (segment (start 110 68.5) (end 106.426 72.074) (width 0.25) (layer B.Cu) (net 34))
 (segment (start 106.426 72.074) (end 106.426 80.264) (width 0.25) (layer B.Cu) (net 34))
 (segment (start 106.426 80.264) (end 105.918 80.772) (width 0.25) (layer B.Cu) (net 34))
 (segment (start 105.918 80.772) (end 104.14 80.772) (width 0.25) (layer B.Cu) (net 34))
 (segment (start 105.918 80.772) (end 108.966 80.772) (width 0.25) (layer B.Cu) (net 34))
 (segment (start 94.234 80.772) (end 94.234 80.772) (width 0.25) (layer B.Cu) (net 34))
 (via (at 94.234 80.772) (size 0.8) (drill 0.4) (layers F.Cu B.Cu) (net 34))
 (segment (start 99.314 80.772) (end 94.234 80.772) (width 0.25) (layer B.Cu) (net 34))
 (via (at 99.314 80.772) (size 0.8) (drill 0.4) (layers F.Cu B.Cu) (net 34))
 (segment (start 104.14 80.772) (end 99.314 80.772) (width 0.25) (layer B.Cu) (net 34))
 (via (at 104.14 80.772) (size 0.8) (drill 0.4) (layers F.Cu B.Cu) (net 34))
 (segment (start 108.966 80.772) (end 113.284 80.772) (width 0.25) (layer B.Cu) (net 34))
 (via (at 108.966 80.772) (size 0.8) (drill 0.4) (layers F.Cu B.Cu) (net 34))
 (segment (start 113.284 80.772) (end 118.11 80.772) (width 0.25) (layer B.Cu) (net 34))
 (via (at 113.284 80.772) (size 0.8) (drill 0.4) (layers F.Cu B.Cu) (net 34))
 (segment (start 118.11 80.772) (end 123.19 80.772) (width 0.25) (layer B.Cu) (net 34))
 (via (at 118.11 80.772) (size 0.8) (drill 0.4) (layers F.Cu B.Cu) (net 34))
 (segment (start 123.19 80.772) (end 128.27 80.772) (width 0.25) (layer B.Cu) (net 34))
 (via (at 123.19 80.772) (size 0.8) (drill 0.4) (layers F.Cu B.Cu) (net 34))
 (segment (start 128.27 80.772) (end 128.27 80.772) (width 0.25) (layer B.Cu) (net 34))
 (via (at 128.27 80.772) (size 0.8) (drill 0.4) (layers F.Cu B.Cu) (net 34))
 (segment (start 94 81.006) (end 94.234 80.772) (width 0.25) (layer F.Cu) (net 34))
 (segment (start 94 82.35) (end 94 81.006) (width 0.25) (layer F.Cu) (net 34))
 (segment (start 99 81.086) (end 99.314 80.772) (width 0.25) (layer F.Cu) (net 34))
 (segment (start 99 82.35) (end 99 81.086) (width 0.25) (layer F.Cu) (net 34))
 (segment (start 104 80.912) (end 104.14 80.772) (width 0.25) (layer F.Cu) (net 34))
 (segment (start 104 82.35) (end 104 80.912) (width 0.25) (layer F.Cu) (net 34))
 (segment (start 109 80.806) (end 108.966 80.772) (width 0.25) (layer F.Cu) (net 34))
 (segment (start 109 82.35) (end 109 80.806) (width 0.25) (layer F.Cu) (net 34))
 (segment (start 114 81.488) (end 113.284 80.772) (width 0.25) (layer F.Cu) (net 34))
 (segment (start 114 82.35) (end 114 81.488) (width 0.25) (layer F.Cu) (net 34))
 (segment (start 119 81.662) (end 118.11 80.772) (width 0.25) (layer F.Cu) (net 34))
 (segment (start 119 82.35) (end 119 81.662) (width 0.25) (layer F.Cu) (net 34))
 (segment (start 124 81.582) (end 123.19 80.772) (width 0.25) (layer F.Cu) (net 34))
 (segment (start 124 82.35) (end 124 81.582) (width 0.25) (layer F.Cu) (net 34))
 (segment (start 129 81.502) (end 128.27 80.772) (width 0.25) (layer F.Cu) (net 34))
 (segment (start 129 82.35) (end 129 81.502) (width 0.25) (layer F.Cu) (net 34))
 (segment (start 111.5 78.5) (end 110 77) (width 0.25) (layer F.Cu) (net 33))
 (segment (start 116.5 81.6) (end 114.9 80) (width 0.25) (layer F.Cu) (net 33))
 (segment (start 114.9 80) (end 111.5 80) (width 0.25) (layer F.Cu) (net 33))
 (segment (start 116.5 82.35) (end 116.5 81.6) (width 0.25) (layer F.Cu) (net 33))
 (segment (start 111.5 80) (end 111.5 78.5) (width 0.25) (layer F.Cu) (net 33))
 (segment (start 111.5 82.35) (end 111.5 80) (width 0.25) (layer F.Cu) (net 33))
 (segment (start 119.9 80) (end 114.9 80) (width 0.25) (layer F.Cu) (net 33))
 (segment (start 121.5 81.6) (end 119.9 80) (width 0.25) (layer F.Cu) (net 33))
 (segment (start 121.5 82.35) (end 121.5 81.6) (width 0.25) (layer F.Cu) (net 33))
 (segment (start 126.5 82.35) (end 126.5 81.5) (width 0.25) (layer F.Cu) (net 33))
 (segment (start 125 80) (end 119.9 80) (width 0.25) (layer F.Cu) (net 33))
 (segment (start 126.5 81.5) (end 125 80) (width 0.25) (layer F.Cu) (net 33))
 (segment (start 106.5 82.35) (end 106.5 81) (width 0.25) (layer F.Cu) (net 33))
 (segment (start 106.5 81) (end 107.5 80) (width 0.25) (layer F.Cu) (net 33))
 (segment (start 107.5 80) (end 111.5 80) (width 0.25) (layer F.Cu) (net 33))
 (segment (start 101.5 81.6) (end 103.1 80) (width 0.25) (layer F.Cu) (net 33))
 (segment (start 101.5 82.35) (end 101.5 81.6) (width 0.25) (layer F.Cu) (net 33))
 (segment (start 103.1 80) (end 107.5 80) (width 0.25) (layer F.Cu) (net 33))
 (segment (start 96.5 81.6) (end 98.1 80) (width 0.25) (layer F.Cu) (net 33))
 (segment (start 96.5 82.35) (end 96.5 81.6) (width 0.25) (layer F.Cu) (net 33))
 (segment (start 98.1 80) (end 103.1 80) (width 0.25) (layer F.Cu) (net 33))
 (segment (start 91.5 81.6) (end 93.1 80) (width 0.25) (layer F.Cu) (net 33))
 (segment (start 91.5 82.35) (end 91.5 81.6) (width 0.25) (layer F.Cu) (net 33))
 (segment (start 93.1 80) (end 98 80) (width 0.25) (layer F.Cu) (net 33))
 (segment (start 91.5 83.65) (end 94 83.65) (width 0.25) (layer F.Cu) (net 25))
 (segment (start 94 87.46) (end 101.5 94.96) (width 0.25) (layer F.Cu) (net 25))
 (segment (start 94 83.65) (end 94 87.46) (width 0.25) (layer F.Cu) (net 25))
 (segment (start 96.5 83.65) (end 99 83.65) (width 0.25) (layer F.Cu) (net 26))
 (segment (start 104.04 93.738686) (end 104.04 94.96) (width 0.25) (layer F.Cu) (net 26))
 (segment (start 99.25 83.65) (end 104.04 88.44) (width 0.25) (layer F.Cu) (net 26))
 (segment (start 104.04 88.44) (end 104.04 93.738686) (width 0.25) (layer F.Cu) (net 26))
 (segment (start 99 83.65) (end 99.25 83.65) (width 0.25) (layer F.Cu) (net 26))
 (segment (start 101.5 83.65) (end 104 83.65) (width 0.25) (layer F.Cu) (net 27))
 (segment (start 106.58 93.738686) (end 106.58 94.96) (width 0.25) (layer F.Cu) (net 27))
 (segment (start 106.58 86.98) (end 106.58 93.738686) (width 0.25) (layer F.Cu) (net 27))
 (segment (start 104 84.4) (end 106.58 86.98) (width 0.25) (layer F.Cu) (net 27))
 (segment (start 104 83.65) (end 104 84.4) (width 0.25) (layer F.Cu) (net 27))
 (segment (start 106.5 83.65) (end 109 83.65) (width 0.25) (layer F.Cu) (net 28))
 (segment (start 109 94.84) (end 109.12 94.96) (width 0.25) (layer F.Cu) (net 28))
 (segment (start 109 83.65) (end 109 94.84) (width 0.25) (layer F.Cu) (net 28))
 (segment (start 114 83.65) (end 111.5 83.65) (width 0.25) (layer F.Cu) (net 29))
 (segment (start 111.5 94.8) (end 111.66 94.96) (width 0.25) (layer F.Cu) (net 29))
 (segment (start 111.5 83.65) (end 111.5 94.8) (width 0.25) (layer F.Cu) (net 29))
 (segment (start 116.25 83.65) (end 116.5 83.65) (width 0.25) (layer F.Cu) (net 30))
 (segment (start 114.2 85.7) (end 116.25 83.65) (width 0.25) (layer F.Cu) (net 30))
 (segment (start 114.2 94.96) (end 114.2 85.7) (width 0.25) (layer F.Cu) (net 30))
 (segment (start 116.5 83.65) (end 119 83.65) (width 0.25) (layer F.Cu) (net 30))
 (segment (start 124 83.65) (end 121.5 83.65) (width 0.25) (layer F.Cu) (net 31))
 (segment (start 116.74 93.738686) (end 116.74 94.96) (width 0.25) (layer F.Cu) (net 31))
 (segment (start 116.74 92.77359) (end 116.74 93.738686) (width 0.25) (layer F.Cu) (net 31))
 (segment (start 121.5 83.65) (end 121.5 88.01359) (width 0.25) (layer F.Cu) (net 31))
 (segment (start 121.5 88.01359) (end 116.74 92.77359) (width 0.25) (layer F.Cu) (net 31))
 (segment (start 119.28 90.87) (end 126.5 83.65) (width 0.25) (layer F.Cu) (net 32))
 (segment (start 119.28 94.96) (end 119.28 90.87) (width 0.25) (layer F.Cu) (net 32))
 (segment (start 129 83.65) (end 126.5 83.65) (width 0.25) (layer F.Cu) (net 32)))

